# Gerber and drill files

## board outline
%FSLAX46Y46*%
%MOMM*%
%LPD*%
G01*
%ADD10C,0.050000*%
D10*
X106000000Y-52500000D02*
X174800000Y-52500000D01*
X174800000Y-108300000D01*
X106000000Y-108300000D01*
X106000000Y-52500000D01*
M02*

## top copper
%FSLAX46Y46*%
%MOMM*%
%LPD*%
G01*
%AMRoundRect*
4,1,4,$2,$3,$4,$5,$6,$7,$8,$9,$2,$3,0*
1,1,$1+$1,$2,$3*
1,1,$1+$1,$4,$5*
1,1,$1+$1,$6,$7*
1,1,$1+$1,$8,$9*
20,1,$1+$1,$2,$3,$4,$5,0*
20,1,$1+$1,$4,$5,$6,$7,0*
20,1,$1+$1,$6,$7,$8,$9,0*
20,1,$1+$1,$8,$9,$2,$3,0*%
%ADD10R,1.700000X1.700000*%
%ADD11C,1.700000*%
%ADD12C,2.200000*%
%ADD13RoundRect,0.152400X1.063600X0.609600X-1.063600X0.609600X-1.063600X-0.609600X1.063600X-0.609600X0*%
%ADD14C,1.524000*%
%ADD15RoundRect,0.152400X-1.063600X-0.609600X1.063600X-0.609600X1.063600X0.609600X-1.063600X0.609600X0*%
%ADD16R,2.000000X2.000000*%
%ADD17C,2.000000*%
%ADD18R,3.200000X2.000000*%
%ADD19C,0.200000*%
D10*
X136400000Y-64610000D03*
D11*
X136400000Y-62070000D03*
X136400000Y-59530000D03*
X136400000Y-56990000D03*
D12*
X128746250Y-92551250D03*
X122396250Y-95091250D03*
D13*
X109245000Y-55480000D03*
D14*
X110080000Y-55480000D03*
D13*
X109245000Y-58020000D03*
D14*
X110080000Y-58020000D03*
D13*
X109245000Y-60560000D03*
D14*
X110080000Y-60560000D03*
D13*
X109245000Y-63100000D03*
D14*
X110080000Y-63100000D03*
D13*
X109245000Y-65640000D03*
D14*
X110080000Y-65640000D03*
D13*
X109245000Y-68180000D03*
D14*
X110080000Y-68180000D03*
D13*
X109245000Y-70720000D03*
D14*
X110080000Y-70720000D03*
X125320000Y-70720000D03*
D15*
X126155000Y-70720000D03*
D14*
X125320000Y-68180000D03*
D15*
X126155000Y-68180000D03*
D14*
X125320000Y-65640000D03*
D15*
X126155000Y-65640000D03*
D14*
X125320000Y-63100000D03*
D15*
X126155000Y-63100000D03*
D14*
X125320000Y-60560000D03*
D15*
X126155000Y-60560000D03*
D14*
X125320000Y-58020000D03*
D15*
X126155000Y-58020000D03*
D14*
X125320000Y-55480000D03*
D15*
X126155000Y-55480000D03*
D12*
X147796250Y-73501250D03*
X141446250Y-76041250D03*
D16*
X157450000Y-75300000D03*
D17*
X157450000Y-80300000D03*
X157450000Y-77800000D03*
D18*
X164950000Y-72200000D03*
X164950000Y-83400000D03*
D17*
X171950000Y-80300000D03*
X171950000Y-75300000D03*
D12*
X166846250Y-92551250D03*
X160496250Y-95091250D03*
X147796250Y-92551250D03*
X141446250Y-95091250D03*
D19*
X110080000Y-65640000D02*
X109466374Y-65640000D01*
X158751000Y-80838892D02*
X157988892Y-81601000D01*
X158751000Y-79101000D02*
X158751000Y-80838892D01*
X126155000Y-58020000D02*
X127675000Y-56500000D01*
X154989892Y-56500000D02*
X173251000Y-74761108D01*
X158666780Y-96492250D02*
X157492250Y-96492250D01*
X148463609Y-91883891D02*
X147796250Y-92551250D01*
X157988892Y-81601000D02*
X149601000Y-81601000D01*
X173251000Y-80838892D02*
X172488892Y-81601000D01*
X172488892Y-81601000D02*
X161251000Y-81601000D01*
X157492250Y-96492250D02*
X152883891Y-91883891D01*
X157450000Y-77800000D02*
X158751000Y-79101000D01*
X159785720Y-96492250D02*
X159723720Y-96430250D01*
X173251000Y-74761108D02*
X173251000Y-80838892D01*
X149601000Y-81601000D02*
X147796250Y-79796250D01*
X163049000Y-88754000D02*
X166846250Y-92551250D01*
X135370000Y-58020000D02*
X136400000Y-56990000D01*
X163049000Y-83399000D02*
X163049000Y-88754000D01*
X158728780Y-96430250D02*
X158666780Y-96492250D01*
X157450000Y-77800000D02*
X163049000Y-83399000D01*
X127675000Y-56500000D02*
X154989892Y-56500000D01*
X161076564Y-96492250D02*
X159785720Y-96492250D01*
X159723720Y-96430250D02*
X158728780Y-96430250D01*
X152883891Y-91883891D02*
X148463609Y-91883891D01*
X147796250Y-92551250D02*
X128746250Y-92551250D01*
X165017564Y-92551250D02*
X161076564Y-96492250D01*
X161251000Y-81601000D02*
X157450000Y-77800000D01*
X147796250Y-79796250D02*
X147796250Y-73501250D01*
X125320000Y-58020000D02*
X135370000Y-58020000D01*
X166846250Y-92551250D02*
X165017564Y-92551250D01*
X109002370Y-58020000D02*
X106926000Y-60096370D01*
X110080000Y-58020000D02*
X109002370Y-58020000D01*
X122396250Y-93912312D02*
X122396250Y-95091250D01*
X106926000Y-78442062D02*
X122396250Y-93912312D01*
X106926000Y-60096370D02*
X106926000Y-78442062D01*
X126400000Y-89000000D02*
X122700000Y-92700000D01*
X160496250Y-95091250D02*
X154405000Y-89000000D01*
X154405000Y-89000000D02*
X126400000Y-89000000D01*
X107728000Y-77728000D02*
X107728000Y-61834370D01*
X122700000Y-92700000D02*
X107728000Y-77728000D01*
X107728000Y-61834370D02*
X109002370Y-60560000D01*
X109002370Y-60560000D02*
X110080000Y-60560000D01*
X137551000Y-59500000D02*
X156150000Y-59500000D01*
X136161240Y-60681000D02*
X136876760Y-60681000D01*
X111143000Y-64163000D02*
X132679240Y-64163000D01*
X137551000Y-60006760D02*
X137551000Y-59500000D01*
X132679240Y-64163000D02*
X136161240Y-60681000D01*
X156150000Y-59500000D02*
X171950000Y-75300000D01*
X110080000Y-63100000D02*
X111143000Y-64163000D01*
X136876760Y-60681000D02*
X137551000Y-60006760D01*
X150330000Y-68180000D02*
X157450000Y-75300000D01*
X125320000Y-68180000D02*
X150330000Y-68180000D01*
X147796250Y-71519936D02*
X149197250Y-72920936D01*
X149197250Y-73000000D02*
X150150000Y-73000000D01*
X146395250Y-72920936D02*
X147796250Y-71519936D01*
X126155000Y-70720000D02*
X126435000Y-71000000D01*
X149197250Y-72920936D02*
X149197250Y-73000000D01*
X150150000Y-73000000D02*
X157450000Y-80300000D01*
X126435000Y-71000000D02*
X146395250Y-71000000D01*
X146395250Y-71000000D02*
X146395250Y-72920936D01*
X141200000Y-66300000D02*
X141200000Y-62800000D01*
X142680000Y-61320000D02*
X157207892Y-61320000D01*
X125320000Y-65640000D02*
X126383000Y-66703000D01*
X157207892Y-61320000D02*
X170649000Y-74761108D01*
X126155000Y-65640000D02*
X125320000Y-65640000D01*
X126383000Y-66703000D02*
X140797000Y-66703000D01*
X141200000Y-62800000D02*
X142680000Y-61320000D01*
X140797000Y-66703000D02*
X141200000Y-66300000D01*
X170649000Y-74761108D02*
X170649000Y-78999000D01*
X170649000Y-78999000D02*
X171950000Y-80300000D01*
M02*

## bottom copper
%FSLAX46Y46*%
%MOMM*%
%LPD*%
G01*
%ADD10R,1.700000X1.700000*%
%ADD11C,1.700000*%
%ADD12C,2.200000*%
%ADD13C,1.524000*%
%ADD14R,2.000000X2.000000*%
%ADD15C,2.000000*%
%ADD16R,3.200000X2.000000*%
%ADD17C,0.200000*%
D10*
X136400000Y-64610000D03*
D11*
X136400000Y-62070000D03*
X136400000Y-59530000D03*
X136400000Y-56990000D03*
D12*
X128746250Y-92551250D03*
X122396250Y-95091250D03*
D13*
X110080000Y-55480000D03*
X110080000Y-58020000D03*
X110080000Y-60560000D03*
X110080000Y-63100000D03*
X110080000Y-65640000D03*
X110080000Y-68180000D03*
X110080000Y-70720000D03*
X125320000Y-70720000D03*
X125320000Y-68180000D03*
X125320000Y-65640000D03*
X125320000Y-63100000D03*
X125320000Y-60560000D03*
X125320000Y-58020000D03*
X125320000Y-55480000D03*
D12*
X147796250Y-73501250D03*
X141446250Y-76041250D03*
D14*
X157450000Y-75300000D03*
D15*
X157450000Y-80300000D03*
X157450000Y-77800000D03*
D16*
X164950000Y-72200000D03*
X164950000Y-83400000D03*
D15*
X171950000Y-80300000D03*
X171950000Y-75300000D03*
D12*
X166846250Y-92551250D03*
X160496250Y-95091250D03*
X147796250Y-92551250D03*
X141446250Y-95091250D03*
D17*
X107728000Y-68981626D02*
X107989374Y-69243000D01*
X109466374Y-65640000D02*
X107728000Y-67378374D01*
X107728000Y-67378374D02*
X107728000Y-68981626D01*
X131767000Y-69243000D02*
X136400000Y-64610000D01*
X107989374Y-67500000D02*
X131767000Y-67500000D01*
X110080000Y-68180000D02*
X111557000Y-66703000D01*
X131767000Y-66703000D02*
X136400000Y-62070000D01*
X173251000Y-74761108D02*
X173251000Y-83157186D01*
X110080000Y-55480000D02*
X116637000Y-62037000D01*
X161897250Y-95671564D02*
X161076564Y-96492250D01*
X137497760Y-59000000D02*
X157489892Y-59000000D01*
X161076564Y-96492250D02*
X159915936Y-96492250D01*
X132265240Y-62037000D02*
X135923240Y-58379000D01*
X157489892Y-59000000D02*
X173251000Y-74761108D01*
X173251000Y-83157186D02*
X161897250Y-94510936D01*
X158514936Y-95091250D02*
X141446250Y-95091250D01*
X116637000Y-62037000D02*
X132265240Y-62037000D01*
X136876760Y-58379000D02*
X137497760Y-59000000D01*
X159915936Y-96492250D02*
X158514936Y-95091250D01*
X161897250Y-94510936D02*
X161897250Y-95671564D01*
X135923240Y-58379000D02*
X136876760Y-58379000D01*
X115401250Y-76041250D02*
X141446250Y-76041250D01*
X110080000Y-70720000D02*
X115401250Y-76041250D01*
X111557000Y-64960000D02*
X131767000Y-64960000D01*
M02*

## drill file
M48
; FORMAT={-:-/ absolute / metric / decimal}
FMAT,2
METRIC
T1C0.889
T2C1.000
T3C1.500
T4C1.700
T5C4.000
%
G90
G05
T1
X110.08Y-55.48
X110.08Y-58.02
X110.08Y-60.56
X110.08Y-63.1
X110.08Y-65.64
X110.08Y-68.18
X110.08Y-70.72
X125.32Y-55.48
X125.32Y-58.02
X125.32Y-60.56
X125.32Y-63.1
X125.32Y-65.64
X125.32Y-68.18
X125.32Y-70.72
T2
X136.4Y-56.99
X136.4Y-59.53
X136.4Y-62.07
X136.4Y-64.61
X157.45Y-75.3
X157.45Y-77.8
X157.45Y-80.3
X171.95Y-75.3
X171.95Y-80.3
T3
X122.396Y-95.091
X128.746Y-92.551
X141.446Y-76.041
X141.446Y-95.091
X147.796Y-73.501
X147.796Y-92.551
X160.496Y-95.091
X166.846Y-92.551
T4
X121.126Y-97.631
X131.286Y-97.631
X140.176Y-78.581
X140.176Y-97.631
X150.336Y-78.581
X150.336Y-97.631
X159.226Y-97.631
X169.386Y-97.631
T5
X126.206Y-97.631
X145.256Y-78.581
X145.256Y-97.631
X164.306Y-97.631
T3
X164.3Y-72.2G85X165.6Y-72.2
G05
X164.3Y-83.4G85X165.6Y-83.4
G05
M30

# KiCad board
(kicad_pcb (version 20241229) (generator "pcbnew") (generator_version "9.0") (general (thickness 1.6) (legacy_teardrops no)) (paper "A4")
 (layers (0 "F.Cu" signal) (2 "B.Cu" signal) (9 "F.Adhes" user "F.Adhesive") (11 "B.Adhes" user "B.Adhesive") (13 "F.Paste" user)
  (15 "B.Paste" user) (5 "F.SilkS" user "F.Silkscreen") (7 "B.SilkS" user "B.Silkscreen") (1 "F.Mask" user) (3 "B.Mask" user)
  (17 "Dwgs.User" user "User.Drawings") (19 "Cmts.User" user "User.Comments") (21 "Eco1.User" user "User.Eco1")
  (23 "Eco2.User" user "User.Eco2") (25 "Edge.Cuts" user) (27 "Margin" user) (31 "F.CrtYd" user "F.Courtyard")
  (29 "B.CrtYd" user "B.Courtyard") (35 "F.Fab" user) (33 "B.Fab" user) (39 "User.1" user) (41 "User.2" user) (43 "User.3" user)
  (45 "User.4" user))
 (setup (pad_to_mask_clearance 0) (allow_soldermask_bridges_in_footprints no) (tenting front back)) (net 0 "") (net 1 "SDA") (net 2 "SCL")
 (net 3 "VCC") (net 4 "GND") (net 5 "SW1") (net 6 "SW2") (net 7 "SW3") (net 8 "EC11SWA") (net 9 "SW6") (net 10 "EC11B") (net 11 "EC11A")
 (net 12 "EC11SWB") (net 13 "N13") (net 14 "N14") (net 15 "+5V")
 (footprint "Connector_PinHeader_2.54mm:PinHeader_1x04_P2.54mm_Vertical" (layer "F.Cu") (at 136.4 64.61 180)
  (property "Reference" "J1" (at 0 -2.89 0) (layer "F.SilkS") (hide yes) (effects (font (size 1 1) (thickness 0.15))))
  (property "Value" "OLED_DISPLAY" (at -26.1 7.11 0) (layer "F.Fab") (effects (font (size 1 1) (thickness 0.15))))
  (pad "1" thru_hole rect (at 0 0 180) (size 1.7 1.7) (drill 1) (layers "*.Cu" "*.Mask") (remove_unused_layers no) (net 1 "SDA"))
  (pad "2" thru_hole circle (at 0 2.54 180) (size 1.7 1.7) (drill 1) (layers "*.Cu" "*.Mask") (remove_unused_layers no) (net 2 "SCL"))
  (pad "3" thru_hole circle (at 0 5.08 180) (size 1.7 1.7) (drill 1) (layers "*.Cu" "*.Mask") (remove_unused_layers no) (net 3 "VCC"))
  (pad "4" thru_hole circle (at 0 7.62 180) (size 1.7 1.7) (drill 1) (layers "*.Cu" "*.Mask") (remove_unused_layers no) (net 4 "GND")))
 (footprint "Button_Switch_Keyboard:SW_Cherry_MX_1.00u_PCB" (layer "F.Cu") (at 128.74625 92.55125)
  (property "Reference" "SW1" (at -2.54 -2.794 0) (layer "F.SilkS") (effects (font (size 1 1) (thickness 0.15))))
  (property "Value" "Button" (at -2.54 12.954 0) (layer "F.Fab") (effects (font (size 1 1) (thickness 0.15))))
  (pad "" np_thru_hole circle (at -7.62 5.08) (size 1.7 1.7) (drill 1.7) (layers "*.Cu" "*.Mask"))
  (pad "" np_thru_hole circle (at -2.54 5.08) (size 4 4) (drill 4) (layers "*.Cu" "*.Mask"))
  (pad "" np_thru_hole circle (at 2.54 5.08) (size 1.7 1.7) (drill 1.7) (layers "*.Cu" "*.Mask"))
  (pad "1" thru_hole circle (at 0 0) (size 2.2 2.2) (drill 1.5) (layers "*.Cu" "*.Mask") (remove_unused_layers no) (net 4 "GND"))
  (pad "2" thru_hole circle (at -6.35 2.54) (size 2.2 2.2) (drill 1.5) (layers "*.Cu" "*.Mask") (remove_unused_layers no) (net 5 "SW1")))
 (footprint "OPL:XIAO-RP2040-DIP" (layer "F.Cu") (at 117.7 63.1)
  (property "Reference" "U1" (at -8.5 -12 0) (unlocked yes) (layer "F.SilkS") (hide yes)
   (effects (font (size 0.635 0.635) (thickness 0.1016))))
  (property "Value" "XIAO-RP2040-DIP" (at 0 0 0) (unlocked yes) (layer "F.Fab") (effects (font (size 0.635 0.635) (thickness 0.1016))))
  (pad "1" smd roundrect (at -8.455 -7.62 180) (size 2.432 1.524) (layers "F.Cu" "F.Mask") (roundrect_rratio 0.1) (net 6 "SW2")
   (thermal_bridge_angle 45))
  (pad "1" thru_hole circle (at -7.62 -7.62 180) (size 1.524 1.524) (drill 0.889) (layers "*.Cu" "*.Mask") (remove_unused_layers no)
   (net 6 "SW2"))
  (pad "2" smd roundrect (at -8.455 -5.08 180) (size 2.432 1.524) (layers "F.Cu" "F.Mask") (roundrect_rratio 0.1) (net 5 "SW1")
   (thermal_bridge_angle 45))
  (pad "2" thru_hole circle (at -7.62 -5.08 180) (size 1.524 1.524) (drill 0.889) (layers "*.Cu" "*.Mask") (remove_unused_layers no)
   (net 5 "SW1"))
  (pad "3" smd roundrect (at -8.455 -2.54 180) (size 2.432 1.524) (layers "F.Cu" "F.Mask") (roundrect_rratio 0.1) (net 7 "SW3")
   (thermal_bridge_angle 45))
  (pad "3" thru_hole circle (at -7.62 -2.54 180) (size 1.524 1.524) (drill 0.889) (layers "*.Cu" "*.Mask") (remove_unused_layers no)
   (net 7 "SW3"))
  (pad "4" smd roundrect (at -8.455 0 180) (size 2.432 1.524) (layers "F.Cu" "F.Mask") (roundrect_rratio 0.1) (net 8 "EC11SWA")
   (thermal_bridge_angle 45))
  (pad "4" thru_hole circle (at -7.62 0 180) (size 1.524 1.524) (drill 0.889) (layers "*.Cu" "*.Mask") (remove_unused_layers no)
   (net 8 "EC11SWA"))
  (pad "5" smd roundrect (at -8.455 2.54 180) (size 2.432 1.524) (layers "F.Cu" "F.Mask") (roundrect_rratio 0.1) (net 1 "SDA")
   (thermal_bridge_angle 45))
  (pad "5" thru_hole circle (at -7.62 2.54 180) (size 1.524 1.524) (drill 0.889) (layers "*.Cu" "*.Mask") (remove_unused_layers no)
   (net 1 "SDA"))
  (pad "6" smd roundrect (at -8.455 5.08 180) (size 2.432 1.524) (layers "F.Cu" "F.Mask") (roundrect_rratio 0.1) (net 2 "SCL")
   (thermal_bridge_angle 45))
  (pad "6" thru_hole circle (at -7.62 5.08 180) (size 1.524 1.524) (drill 0.889) (layers "*.Cu" "*.Mask") (remove_unused_layers no)
   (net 2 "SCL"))
  (pad "7" smd roundrect (at -8.455 7.62 180) (size 2.432 1.524) (layers "F.Cu" "F.Mask") (roundrect_rratio 0.1) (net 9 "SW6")
   (thermal_bridge_angle 45))
  (pad "7" thru_hole circle (at -7.62 7.62 180) (size 1.524 1.524) (drill 0.889) (layers "*.Cu" "*.Mask") (remove_unused_layers no)
   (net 9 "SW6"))
  (pad "8" thru_hole circle (at 7.62 7.62) (size 1.524 1.524) (drill 0.889) (layers "*.Cu" "*.Mask") (remove_unused_layers no)
   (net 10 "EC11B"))
  (pad "8" smd roundrect (at 8.455 7.62) (size 2.432 1.524) (layers "F.Cu" "F.Mask") (roundrect_rratio 0.1) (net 10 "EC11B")
   (thermal_bridge_angle 45))
  (pad "9" thru_hole circle (at 7.62 5.08) (size 1.524 1.524) (drill 0.889) (layers "*.Cu" "*.Mask") (remove_unused_layers no)
   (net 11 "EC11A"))
  (pad "9" smd roundrect (at 8.455 5.08) (size 2.432 1.524) (layers "F.Cu" "F.Mask") (roundrect_rratio 0.1) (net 11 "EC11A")
   (thermal_bridge_angle 45))
  (pad "10" thru_hole circle (at 7.62 2.54) (size 1.524 1.524) (drill 0.889) (layers "*.Cu" "*.Mask") (remove_unused_layers no)
   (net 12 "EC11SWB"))
  (pad "10" smd roundrect (at 8.455 2.54) (size 2.432 1.524) (layers "F.Cu" "F.Mask") (roundrect_rratio 0.1) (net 12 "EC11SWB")
   (thermal_bridge_angle 45))
  (pad "11" thru_hole circle (at 7.62 0) (size 1.524 1.524) (drill 0.889) (layers "*.Cu" "*.Mask") (remove_unused_layers no) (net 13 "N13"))
  (pad "11" smd roundrect (at 8.455 0) (size 2.432 1.524) (layers "F.Cu" "F.Mask") (roundrect_rratio 0.1) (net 13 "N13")
   (thermal_bridge_angle 45))
  (pad "12" thru_hole circle (at 7.62 -2.54) (size 1.524 1.524) (drill 0.889) (layers "*.Cu" "*.Mask") (remove_unused_layers no)
   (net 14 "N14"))
  (pad "12" smd roundrect (at 8.455 -2.54) (size 2.432 1.524) (layers "F.Cu" "F.Mask") (roundrect_rratio 0.1) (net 14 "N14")
   (thermal_bridge_angle 45))
  (pad "13" thru_hole circle (at 7.62 -5.08) (size 1.524 1.524) (drill 0.889) (layers "*.Cu" "*.Mask") (remove_unused_layers no)
   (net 4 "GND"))
  (pad "13" smd roundrect (at 8.455 -5.08) (size 2.432 1.524) (layers "F.Cu" "F.Mask") (roundrect_rratio 0.1) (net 4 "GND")
   (thermal_bridge_angle 45))
  (pad "14" thru_hole circle (at 7.62 -7.62) (size 1.524 1.524) (drill 0.889) (layers "*.Cu" "*.Mask") (remove_unused_layers no)
   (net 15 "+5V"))
  (pad "14" smd roundrect (at 8.455 -7.62) (size 2.432 1.524) (layers "F.Cu" "F.Mask") (roundrect_rratio 0.1) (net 15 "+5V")
   (thermal_bridge_angle 45)))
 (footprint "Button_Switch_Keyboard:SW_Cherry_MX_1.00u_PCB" (layer "F.Cu") (at 147.79625 73.50125)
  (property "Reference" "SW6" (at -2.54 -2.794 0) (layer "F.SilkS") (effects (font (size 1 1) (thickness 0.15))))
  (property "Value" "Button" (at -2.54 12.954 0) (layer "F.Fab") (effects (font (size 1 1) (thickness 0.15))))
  (pad "" np_thru_hole circle (at -7.62 5.08) (size 1.7 1.7) (drill 1.7) (layers "*.Cu" "*.Mask"))
  (pad "" np_thru_hole circle (at -2.54 5.08) (size 4 4) (drill 4) (layers "*.Cu" "*.Mask"))
  (pad "" np_thru_hole circle (at 2.54 5.08) (size 1.7 1.7) (drill 1.7) (layers "*.Cu" "*.Mask"))
  (pad "1" thru_hole circle (at 0 0) (size 2.2 2.2) (drill 1.5) (layers "*.Cu" "*.Mask") (remove_unused_layers no) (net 4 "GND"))
  (pad "2" thru_hole circle (at -6.35 2.54) (size 2.2 2.2) (drill 1.5) (layers "*.Cu" "*.Mask") (remove_unused_layers no) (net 9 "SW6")))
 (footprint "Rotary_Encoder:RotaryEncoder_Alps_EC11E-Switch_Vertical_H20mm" (layer "F.Cu") (at 157.45 75.3)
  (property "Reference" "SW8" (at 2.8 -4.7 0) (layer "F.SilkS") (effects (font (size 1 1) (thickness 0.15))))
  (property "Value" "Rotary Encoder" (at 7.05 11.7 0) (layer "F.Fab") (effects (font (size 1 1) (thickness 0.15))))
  (pad "A" thru_hole rect (at 0 0) (size 2 2) (drill 1) (layers "*.Cu" "*.Mask") (remove_unused_layers no) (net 11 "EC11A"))
  (pad "B" thru_hole circle (at 0 5) (size 2 2) (drill 1) (layers "*.Cu" "*.Mask") (remove_unused_layers no) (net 10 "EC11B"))
  (pad "C" thru_hole circle (at 0 2.5) (size 2 2) (drill 1) (layers "*.Cu" "*.Mask") (remove_unused_layers no) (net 4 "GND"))
  (pad "MP" thru_hole rect (at 7.5 -3.1) (size 3.2 2) (drill oval 2.8 1.5) (layers "*.Cu" "*.Mask") (remove_unused_layers no))
  (pad "MP" thru_hole rect (at 7.5 8.1) (size 3.2 2) (drill oval 2.8 1.5) (layers "*.Cu" "*.Mask") (remove_unused_layers no))
  (pad "S1" thru_hole circle (at 14.5 5) (size 2 2) (drill 1) (layers "*.Cu" "*.Mask") (remove_unused_layers no) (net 12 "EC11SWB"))
  (pad "S2" thru_hole circle (at 14.5 0) (size 2 2) (drill 1) (layers "*.Cu" "*.Mask") (remove_unused_layers no) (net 8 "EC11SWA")))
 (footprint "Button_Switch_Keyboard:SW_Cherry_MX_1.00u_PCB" (layer "F.Cu") (at 166.84625 92.55125)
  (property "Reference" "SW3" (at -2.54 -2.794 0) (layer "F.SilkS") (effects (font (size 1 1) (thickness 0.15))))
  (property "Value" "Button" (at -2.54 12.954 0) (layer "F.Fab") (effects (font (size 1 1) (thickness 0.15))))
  (pad "" np_thru_hole circle (at -7.62 5.08) (size 1.7 1.7) (drill 1.7) (layers "*.Cu" "*.Mask"))
  (pad "" np_thru_hole circle (at -2.54 5.08) (size 4 4) (drill 4) (layers "*.Cu" "*.Mask"))
  (pad "" np_thru_hole circle (at 2.54 5.08) (size 1.7 1.7) (drill 1.7) (layers "*.Cu" "*.Mask"))
  (pad "1" thru_hole circle (at 0 0) (size 2.2 2.2) (drill 1.5) (layers "*.Cu" "*.Mask") (remove_unused_layers no) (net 4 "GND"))
  (pad "2" thru_hole circle (at -6.35 2.54) (size 2.2 2.2) (drill 1.5) (layers "*.Cu" "*.Mask") (remove_unused_layers no) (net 7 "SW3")))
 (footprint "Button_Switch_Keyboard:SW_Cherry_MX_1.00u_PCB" (layer "F.Cu") (at 147.79625 92.55125)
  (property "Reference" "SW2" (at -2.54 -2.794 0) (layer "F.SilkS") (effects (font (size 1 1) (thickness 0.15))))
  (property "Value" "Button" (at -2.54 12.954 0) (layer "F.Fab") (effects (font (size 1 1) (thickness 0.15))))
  (pad "" np_thru_hole circle (at -7.62 5.08) (size 1.7 1.7) (drill 1.7) (layers "*.Cu" "*.Mask"))
  (pad "" np_thru_hole circle (at -2.54 5.08) (size 4 4) (drill 4) (layers "*.Cu" "*.Mask"))
  (pad "" np_thru_hole circle (at 2.54 5.08) (size 1.7 1.7) (drill 1.7) (layers "*.Cu" "*.Mask"))
  (pad "1" thru_hole circle (at 0 0) (size 2.2 2.2) (drill 1.5) (layers "*.Cu" "*.Mask") (remove_unused_layers no) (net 4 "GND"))
  (pad "2" thru_hole circle (at -6.35 2.54) (size 2.2 2.2) (drill 1.5) (layers "*.Cu" "*.Mask") (remove_unused_layers no) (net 6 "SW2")))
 (gr_rect (start 106 52.5) (end 174.8 108.3) (stroke (width 0.05) (type default)) (fill no) (layer "Edge.Cuts"))
 (segment (start 110.08 65.64) (end 109.466374 65.64) (width 0.2) (layer "F.Cu") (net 1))
 (segment (start 107.728 68.981626) (end 107.989374 69.243) (width 0.2) (layer "B.Cu") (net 1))
 (segment (start 109.466374 65.64) (end 107.728 67.378374) (width 0.2) (layer "B.Cu") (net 1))
 (segment (start 107.728 67.378374) (end 107.728 68.981626) (width 0.2) (layer "B.Cu") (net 1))
 (segment (start 131.767 69.243) (end 136.4 64.61) (width 0.2) (layer "B.Cu") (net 1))
 (segment (start 107.989374 67.5) (end 131.767 67.5) (width 0.2) (layer "B.Cu") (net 1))
 (segment (start 110.08 68.18) (end 111.557 66.703) (width 0.2) (layer "B.Cu") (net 2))
 (segment (start 131.767 66.703) (end 136.4 62.07) (width 0.2) (layer "B.Cu") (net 2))
 (segment (start 158.751 80.838892) (end 157.988892 81.601) (width 0.2) (layer "F.Cu") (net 4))
 (segment (start 158.751 79.101) (end 158.751 80.838892) (width 0.2) (layer "F.Cu") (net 4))
 (segment (start 126.155 58.02) (end 127.675 56.5) (width 0.2) (layer "F.Cu") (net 4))
 (segment (start 154.989892 56.5) (end 173.251 74.761108) (width 0.2) (layer "F.Cu") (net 4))
 (segment (start 158.66678 96.49225) (end 157.49225 96.49225) (width 0.2) (layer "F.Cu") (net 4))
 (segment (start 148.463609 91.883891) (end 147.79625 92.55125) (width 0.2) (layer "F.Cu") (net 4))
 (segment (start 157.988892 81.601) (end 149.601 81.601) (width 0.2) (layer "F.Cu") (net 4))
 (segment (start 173.251 80.838892) (end 172.488892 81.601) (width 0.2) (layer "F.Cu") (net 4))
 (segment (start 172.488892 81.601) (end 161.251 81.601) (width 0.2) (layer "F.Cu") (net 4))
 (segment (start 157.49225 96.49225) (end 152.883891 91.883891) (width 0.2) (layer "F.Cu") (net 4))
 (segment (start 157.45 77.8) (end 158.751 79.101) (width 0.2) (layer "F.Cu") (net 4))
 (segment (start 159.78572 96.49225) (end 159.72372 96.43025) (width 0.2) (layer "F.Cu") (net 4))
 (segment (start 173.251 74.761108) (end 173.251 80.838892) (width 0.2) (layer "F.Cu") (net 4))
 (segment (start 149.601 81.601) (end 147.79625 79.79625) (width 0.2) (layer "F.Cu") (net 4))
 (segment (start 163.049 88.754) (end 166.84625 92.55125) (width 0.2) (layer "F.Cu") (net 4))
 (segment (start 135.37 58.02) (end 136.4 56.99) (width 0.2) (layer "F.Cu") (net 4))
 (segment (start 163.049 83.399) (end 163.049 88.754) (width 0.2) (layer "F.Cu") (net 4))
 (segment (start 158.72878 96.43025) (end 158.66678 96.49225) (width 0.2) (layer "F.Cu") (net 4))
 (segment (start 157.45 77.8) (end 163.049 83.399) (width 0.2) (layer "F.Cu") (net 4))
 (segment (start 127.675 56.5) (end 154.989892 56.5) (width 0.2) (layer "F.Cu") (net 4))
 (segment (start 161.076564 96.49225) (end 159.78572 96.49225) (width 0.2) (layer "F.Cu") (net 4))
 (segment (start 159.72372 96.43025) (end 158.72878 96.43025) (width 0.2) (layer "F.Cu") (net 4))
 (segment (start 152.883891 91.883891) (end 148.463609 91.883891) (width 0.2) (layer "F.Cu") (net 4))
 (segment (start 147.79625 92.55125) (end 128.74625 92.55125) (width 0.2) (layer "F.Cu") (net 4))
 (segment (start 165.017564 92.55125) (end 161.076564 96.49225) (width 0.2) (layer "F.Cu") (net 4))
 (segment (start 161.251 81.601) (end 157.45 77.8) (width 0.2) (layer "F.Cu") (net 4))
 (segment (start 147.79625 79.79625) (end 147.79625 73.50125) (width 0.2) (layer "F.Cu") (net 4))
 (segment (start 125.32 58.02) (end 135.37 58.02) (width 0.2) (layer "F.Cu") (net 4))
 (segment (start 166.84625 92.55125) (end 165.017564 92.55125) (width 0.2) (layer "F.Cu") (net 4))
 (segment (start 109.00237 58.02) (end 106.926 60.09637) (width 0.2) (layer "F.Cu") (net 5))
 (segment (start 110.08 58.02) (end 109.00237 58.02) (width 0.2) (layer "F.Cu") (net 5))
 (segment (start 122.39625 93.912312) (end 122.39625 95.09125) (width 0.2) (layer "F.Cu") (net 5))
 (segment (start 106.926 78.442062) (end 122.39625 93.912312) (width 0.2) (layer "F.Cu") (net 5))
 (segment (start 106.926 60.09637) (end 106.926 78.442062) (width 0.2) (layer "F.Cu") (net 5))
 (segment (start 173.251 74.761108) (end 173.251 83.157186) (width 0.2) (layer "B.Cu") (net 6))
 (segment (start 110.08 55.48) (end 116.637 62.037) (width 0.2) (layer "B.Cu") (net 6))
 (segment (start 161.89725 95.671564) (end 161.076564 96.49225) (width 0.2) (layer "B.Cu") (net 6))
 (segment (start 137.49776 59) (end 157.489892 59) (width 0.2) (layer "B.Cu") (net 6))
 (segment (start 161.076564 96.49225) (end 159.915936 96.49225) (width 0.2) (layer "B.Cu") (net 6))
 (segment (start 132.26524 62.037) (end 135.92324 58.379) (width 0.2) (layer "B.Cu") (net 6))
 (segment (start 157.489892 59) (end 173.251 74.761108) (width 0.2) (layer "B.Cu") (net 6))
 (segment (start 173.251 83.157186) (end 161.89725 94.510936) (width 0.2) (layer "B.Cu") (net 6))
 (segment (start 158.514936 95.09125) (end 141.44625 95.09125) (width 0.2) (layer "B.Cu") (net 6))
 (segment (start 116.637 62.037) (end 132.26524 62.037) (width 0.2) (layer "B.Cu") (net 6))
 (segment (start 136.87676 58.379) (end 137.49776 59) (width 0.2) (layer "B.Cu") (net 6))
 (segment (start 159.915936 96.49225) (end 158.514936 95.09125) (width 0.2) (layer "B.Cu") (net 6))
 (segment (start 161.89725 94.510936) (end 161.89725 95.671564) (width 0.2) (layer "B.Cu") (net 6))
 (segment (start 135.92324 58.379) (end 136.87676 58.379) (width 0.2) (layer "B.Cu") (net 6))
 (segment (start 126.4 89) (end 122.7 92.7) (width 0.2) (layer "F.Cu") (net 7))
 (segment (start 160.49625 95.09125) (end 154.405 89) (width 0.2) (layer "F.Cu") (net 7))
 (segment (start 154.405 89) (end 126.4 89) (width 0.2) (layer "F.Cu") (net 7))
 (segment (start 107.728 77.728) (end 107.728 61.83437) (width 0.2) (layer "F.Cu") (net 7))
 (segment (start 122.7 92.7) (end 107.728 77.728) (width 0.2) (layer "F.Cu") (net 7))
 (segment (start 107.728 61.83437) (end 109.00237 60.56) (width 0.2) (layer "F.Cu") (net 7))
 (segment (start 109.00237 60.56) (end 110.08 60.56) (width 0.2) (layer "F.Cu") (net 7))
 (segment (start 115.40125 76.04125) (end 141.44625 76.04125) (width 0.2) (layer "B.Cu") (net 9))
 (segment (start 110.08 70.72) (end 115.40125 76.04125) (width 0.2) (layer "B.Cu") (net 9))
 (segment (start 137.551 59.5) (end 156.15 59.5) (width 0.2) (layer "F.Cu") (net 8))
 (segment (start 136.16124 60.681) (end 136.87676 60.681) (width 0.2) (layer "F.Cu") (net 8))
 (segment (start 111.143 64.163) (end 132.67924 64.163) (width 0.2) (layer "F.Cu") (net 8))
 (segment (start 137.551 60.00676) (end 137.551 59.5) (width 0.2) (layer "F.Cu") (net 8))
 (segment (start 132.67924 64.163) (end 136.16124 60.681) (width 0.2) (layer "F.Cu") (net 8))
 (segment (start 156.15 59.5) (end 171.95 75.3) (width 0.2) (layer "F.Cu") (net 8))
 (segment (start 110.08 63.1) (end 111.143 64.163) (width 0.2) (layer "F.Cu") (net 8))
 (segment (start 136.87676 60.681) (end 137.551 60.00676) (width 0.2) (layer "F.Cu") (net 8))
 (segment (start 150.33 68.18) (end 157.45 75.3) (width 0.2) (layer "F.Cu") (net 11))
 (segment (start 125.32 68.18) (end 150.33 68.18) (width 0.2) (layer "F.Cu") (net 11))
 (segment (start 147.79625 71.519936) (end 149.19725 72.920936) (width 0.2) (layer "F.Cu") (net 10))
 (segment (start 149.19725 73) (end 150.15 73) (width 0.2) (layer "F.Cu") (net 10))
 (segment (start 146.39525 72.920936) (end 147.79625 71.519936) (width 0.2) (layer "F.Cu") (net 10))
 (segment (start 126.155 70.72) (end 126.435 71) (width 0.2) (layer "F.Cu") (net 10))
 (segment (start 149.19725 72.920936) (end 149.19725 73) (width 0.2) (layer "F.Cu") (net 10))
 (segment (start 150.15 73) (end 157.45 80.3) (width 0.2) (layer "F.Cu") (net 10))
 (segment (start 126.435 71) (end 146.39525 71) (width 0.2) (layer "F.Cu") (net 10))
 (segment (start 146.39525 71) (end 146.39525 72.920936) (width 0.2) (layer "F.Cu") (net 10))
 (segment (start 141.2 66.3) (end 141.2 62.8) (width 0.2) (layer "F.Cu") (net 12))
 (segment (start 142.68 61.32) (end 157.207892 61.32) (width 0.2) (layer "F.Cu") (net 12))
 (segment (start 125.32 65.64) (end 126.383 66.703) (width 0.2) (layer "F.Cu") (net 12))
 (segment (start 157.207892 61.32) (end 170.649 74.761108) (width 0.2) (layer "F.Cu") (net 12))
 (segment (start 126.155 65.64) (end 125.32 65.64) (width 0.2) (layer "F.Cu") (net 12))
 (segment (start 126.383 66.703) (end 140.797 66.703) (width 0.2) (layer "F.Cu") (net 12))
 (segment (start 141.2 62.8) (end 142.68 61.32) (width 0.2) (layer "F.Cu") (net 12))
 (segment (start 140.797 66.703) (end 141.2 66.3) (width 0.2) (layer "F.Cu") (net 12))
 (segment (start 170.649 74.761108) (end 170.649 78.999) (width 0.2) (layer "F.Cu") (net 12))
 (segment (start 170.649 78.999) (end 171.95 80.3) (width 0.2) (layer "F.Cu") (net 12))
 (segment (start 111.557 64.96) (end 131.767 64.96) (width 0.2) (layer "B.Cu") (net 12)))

